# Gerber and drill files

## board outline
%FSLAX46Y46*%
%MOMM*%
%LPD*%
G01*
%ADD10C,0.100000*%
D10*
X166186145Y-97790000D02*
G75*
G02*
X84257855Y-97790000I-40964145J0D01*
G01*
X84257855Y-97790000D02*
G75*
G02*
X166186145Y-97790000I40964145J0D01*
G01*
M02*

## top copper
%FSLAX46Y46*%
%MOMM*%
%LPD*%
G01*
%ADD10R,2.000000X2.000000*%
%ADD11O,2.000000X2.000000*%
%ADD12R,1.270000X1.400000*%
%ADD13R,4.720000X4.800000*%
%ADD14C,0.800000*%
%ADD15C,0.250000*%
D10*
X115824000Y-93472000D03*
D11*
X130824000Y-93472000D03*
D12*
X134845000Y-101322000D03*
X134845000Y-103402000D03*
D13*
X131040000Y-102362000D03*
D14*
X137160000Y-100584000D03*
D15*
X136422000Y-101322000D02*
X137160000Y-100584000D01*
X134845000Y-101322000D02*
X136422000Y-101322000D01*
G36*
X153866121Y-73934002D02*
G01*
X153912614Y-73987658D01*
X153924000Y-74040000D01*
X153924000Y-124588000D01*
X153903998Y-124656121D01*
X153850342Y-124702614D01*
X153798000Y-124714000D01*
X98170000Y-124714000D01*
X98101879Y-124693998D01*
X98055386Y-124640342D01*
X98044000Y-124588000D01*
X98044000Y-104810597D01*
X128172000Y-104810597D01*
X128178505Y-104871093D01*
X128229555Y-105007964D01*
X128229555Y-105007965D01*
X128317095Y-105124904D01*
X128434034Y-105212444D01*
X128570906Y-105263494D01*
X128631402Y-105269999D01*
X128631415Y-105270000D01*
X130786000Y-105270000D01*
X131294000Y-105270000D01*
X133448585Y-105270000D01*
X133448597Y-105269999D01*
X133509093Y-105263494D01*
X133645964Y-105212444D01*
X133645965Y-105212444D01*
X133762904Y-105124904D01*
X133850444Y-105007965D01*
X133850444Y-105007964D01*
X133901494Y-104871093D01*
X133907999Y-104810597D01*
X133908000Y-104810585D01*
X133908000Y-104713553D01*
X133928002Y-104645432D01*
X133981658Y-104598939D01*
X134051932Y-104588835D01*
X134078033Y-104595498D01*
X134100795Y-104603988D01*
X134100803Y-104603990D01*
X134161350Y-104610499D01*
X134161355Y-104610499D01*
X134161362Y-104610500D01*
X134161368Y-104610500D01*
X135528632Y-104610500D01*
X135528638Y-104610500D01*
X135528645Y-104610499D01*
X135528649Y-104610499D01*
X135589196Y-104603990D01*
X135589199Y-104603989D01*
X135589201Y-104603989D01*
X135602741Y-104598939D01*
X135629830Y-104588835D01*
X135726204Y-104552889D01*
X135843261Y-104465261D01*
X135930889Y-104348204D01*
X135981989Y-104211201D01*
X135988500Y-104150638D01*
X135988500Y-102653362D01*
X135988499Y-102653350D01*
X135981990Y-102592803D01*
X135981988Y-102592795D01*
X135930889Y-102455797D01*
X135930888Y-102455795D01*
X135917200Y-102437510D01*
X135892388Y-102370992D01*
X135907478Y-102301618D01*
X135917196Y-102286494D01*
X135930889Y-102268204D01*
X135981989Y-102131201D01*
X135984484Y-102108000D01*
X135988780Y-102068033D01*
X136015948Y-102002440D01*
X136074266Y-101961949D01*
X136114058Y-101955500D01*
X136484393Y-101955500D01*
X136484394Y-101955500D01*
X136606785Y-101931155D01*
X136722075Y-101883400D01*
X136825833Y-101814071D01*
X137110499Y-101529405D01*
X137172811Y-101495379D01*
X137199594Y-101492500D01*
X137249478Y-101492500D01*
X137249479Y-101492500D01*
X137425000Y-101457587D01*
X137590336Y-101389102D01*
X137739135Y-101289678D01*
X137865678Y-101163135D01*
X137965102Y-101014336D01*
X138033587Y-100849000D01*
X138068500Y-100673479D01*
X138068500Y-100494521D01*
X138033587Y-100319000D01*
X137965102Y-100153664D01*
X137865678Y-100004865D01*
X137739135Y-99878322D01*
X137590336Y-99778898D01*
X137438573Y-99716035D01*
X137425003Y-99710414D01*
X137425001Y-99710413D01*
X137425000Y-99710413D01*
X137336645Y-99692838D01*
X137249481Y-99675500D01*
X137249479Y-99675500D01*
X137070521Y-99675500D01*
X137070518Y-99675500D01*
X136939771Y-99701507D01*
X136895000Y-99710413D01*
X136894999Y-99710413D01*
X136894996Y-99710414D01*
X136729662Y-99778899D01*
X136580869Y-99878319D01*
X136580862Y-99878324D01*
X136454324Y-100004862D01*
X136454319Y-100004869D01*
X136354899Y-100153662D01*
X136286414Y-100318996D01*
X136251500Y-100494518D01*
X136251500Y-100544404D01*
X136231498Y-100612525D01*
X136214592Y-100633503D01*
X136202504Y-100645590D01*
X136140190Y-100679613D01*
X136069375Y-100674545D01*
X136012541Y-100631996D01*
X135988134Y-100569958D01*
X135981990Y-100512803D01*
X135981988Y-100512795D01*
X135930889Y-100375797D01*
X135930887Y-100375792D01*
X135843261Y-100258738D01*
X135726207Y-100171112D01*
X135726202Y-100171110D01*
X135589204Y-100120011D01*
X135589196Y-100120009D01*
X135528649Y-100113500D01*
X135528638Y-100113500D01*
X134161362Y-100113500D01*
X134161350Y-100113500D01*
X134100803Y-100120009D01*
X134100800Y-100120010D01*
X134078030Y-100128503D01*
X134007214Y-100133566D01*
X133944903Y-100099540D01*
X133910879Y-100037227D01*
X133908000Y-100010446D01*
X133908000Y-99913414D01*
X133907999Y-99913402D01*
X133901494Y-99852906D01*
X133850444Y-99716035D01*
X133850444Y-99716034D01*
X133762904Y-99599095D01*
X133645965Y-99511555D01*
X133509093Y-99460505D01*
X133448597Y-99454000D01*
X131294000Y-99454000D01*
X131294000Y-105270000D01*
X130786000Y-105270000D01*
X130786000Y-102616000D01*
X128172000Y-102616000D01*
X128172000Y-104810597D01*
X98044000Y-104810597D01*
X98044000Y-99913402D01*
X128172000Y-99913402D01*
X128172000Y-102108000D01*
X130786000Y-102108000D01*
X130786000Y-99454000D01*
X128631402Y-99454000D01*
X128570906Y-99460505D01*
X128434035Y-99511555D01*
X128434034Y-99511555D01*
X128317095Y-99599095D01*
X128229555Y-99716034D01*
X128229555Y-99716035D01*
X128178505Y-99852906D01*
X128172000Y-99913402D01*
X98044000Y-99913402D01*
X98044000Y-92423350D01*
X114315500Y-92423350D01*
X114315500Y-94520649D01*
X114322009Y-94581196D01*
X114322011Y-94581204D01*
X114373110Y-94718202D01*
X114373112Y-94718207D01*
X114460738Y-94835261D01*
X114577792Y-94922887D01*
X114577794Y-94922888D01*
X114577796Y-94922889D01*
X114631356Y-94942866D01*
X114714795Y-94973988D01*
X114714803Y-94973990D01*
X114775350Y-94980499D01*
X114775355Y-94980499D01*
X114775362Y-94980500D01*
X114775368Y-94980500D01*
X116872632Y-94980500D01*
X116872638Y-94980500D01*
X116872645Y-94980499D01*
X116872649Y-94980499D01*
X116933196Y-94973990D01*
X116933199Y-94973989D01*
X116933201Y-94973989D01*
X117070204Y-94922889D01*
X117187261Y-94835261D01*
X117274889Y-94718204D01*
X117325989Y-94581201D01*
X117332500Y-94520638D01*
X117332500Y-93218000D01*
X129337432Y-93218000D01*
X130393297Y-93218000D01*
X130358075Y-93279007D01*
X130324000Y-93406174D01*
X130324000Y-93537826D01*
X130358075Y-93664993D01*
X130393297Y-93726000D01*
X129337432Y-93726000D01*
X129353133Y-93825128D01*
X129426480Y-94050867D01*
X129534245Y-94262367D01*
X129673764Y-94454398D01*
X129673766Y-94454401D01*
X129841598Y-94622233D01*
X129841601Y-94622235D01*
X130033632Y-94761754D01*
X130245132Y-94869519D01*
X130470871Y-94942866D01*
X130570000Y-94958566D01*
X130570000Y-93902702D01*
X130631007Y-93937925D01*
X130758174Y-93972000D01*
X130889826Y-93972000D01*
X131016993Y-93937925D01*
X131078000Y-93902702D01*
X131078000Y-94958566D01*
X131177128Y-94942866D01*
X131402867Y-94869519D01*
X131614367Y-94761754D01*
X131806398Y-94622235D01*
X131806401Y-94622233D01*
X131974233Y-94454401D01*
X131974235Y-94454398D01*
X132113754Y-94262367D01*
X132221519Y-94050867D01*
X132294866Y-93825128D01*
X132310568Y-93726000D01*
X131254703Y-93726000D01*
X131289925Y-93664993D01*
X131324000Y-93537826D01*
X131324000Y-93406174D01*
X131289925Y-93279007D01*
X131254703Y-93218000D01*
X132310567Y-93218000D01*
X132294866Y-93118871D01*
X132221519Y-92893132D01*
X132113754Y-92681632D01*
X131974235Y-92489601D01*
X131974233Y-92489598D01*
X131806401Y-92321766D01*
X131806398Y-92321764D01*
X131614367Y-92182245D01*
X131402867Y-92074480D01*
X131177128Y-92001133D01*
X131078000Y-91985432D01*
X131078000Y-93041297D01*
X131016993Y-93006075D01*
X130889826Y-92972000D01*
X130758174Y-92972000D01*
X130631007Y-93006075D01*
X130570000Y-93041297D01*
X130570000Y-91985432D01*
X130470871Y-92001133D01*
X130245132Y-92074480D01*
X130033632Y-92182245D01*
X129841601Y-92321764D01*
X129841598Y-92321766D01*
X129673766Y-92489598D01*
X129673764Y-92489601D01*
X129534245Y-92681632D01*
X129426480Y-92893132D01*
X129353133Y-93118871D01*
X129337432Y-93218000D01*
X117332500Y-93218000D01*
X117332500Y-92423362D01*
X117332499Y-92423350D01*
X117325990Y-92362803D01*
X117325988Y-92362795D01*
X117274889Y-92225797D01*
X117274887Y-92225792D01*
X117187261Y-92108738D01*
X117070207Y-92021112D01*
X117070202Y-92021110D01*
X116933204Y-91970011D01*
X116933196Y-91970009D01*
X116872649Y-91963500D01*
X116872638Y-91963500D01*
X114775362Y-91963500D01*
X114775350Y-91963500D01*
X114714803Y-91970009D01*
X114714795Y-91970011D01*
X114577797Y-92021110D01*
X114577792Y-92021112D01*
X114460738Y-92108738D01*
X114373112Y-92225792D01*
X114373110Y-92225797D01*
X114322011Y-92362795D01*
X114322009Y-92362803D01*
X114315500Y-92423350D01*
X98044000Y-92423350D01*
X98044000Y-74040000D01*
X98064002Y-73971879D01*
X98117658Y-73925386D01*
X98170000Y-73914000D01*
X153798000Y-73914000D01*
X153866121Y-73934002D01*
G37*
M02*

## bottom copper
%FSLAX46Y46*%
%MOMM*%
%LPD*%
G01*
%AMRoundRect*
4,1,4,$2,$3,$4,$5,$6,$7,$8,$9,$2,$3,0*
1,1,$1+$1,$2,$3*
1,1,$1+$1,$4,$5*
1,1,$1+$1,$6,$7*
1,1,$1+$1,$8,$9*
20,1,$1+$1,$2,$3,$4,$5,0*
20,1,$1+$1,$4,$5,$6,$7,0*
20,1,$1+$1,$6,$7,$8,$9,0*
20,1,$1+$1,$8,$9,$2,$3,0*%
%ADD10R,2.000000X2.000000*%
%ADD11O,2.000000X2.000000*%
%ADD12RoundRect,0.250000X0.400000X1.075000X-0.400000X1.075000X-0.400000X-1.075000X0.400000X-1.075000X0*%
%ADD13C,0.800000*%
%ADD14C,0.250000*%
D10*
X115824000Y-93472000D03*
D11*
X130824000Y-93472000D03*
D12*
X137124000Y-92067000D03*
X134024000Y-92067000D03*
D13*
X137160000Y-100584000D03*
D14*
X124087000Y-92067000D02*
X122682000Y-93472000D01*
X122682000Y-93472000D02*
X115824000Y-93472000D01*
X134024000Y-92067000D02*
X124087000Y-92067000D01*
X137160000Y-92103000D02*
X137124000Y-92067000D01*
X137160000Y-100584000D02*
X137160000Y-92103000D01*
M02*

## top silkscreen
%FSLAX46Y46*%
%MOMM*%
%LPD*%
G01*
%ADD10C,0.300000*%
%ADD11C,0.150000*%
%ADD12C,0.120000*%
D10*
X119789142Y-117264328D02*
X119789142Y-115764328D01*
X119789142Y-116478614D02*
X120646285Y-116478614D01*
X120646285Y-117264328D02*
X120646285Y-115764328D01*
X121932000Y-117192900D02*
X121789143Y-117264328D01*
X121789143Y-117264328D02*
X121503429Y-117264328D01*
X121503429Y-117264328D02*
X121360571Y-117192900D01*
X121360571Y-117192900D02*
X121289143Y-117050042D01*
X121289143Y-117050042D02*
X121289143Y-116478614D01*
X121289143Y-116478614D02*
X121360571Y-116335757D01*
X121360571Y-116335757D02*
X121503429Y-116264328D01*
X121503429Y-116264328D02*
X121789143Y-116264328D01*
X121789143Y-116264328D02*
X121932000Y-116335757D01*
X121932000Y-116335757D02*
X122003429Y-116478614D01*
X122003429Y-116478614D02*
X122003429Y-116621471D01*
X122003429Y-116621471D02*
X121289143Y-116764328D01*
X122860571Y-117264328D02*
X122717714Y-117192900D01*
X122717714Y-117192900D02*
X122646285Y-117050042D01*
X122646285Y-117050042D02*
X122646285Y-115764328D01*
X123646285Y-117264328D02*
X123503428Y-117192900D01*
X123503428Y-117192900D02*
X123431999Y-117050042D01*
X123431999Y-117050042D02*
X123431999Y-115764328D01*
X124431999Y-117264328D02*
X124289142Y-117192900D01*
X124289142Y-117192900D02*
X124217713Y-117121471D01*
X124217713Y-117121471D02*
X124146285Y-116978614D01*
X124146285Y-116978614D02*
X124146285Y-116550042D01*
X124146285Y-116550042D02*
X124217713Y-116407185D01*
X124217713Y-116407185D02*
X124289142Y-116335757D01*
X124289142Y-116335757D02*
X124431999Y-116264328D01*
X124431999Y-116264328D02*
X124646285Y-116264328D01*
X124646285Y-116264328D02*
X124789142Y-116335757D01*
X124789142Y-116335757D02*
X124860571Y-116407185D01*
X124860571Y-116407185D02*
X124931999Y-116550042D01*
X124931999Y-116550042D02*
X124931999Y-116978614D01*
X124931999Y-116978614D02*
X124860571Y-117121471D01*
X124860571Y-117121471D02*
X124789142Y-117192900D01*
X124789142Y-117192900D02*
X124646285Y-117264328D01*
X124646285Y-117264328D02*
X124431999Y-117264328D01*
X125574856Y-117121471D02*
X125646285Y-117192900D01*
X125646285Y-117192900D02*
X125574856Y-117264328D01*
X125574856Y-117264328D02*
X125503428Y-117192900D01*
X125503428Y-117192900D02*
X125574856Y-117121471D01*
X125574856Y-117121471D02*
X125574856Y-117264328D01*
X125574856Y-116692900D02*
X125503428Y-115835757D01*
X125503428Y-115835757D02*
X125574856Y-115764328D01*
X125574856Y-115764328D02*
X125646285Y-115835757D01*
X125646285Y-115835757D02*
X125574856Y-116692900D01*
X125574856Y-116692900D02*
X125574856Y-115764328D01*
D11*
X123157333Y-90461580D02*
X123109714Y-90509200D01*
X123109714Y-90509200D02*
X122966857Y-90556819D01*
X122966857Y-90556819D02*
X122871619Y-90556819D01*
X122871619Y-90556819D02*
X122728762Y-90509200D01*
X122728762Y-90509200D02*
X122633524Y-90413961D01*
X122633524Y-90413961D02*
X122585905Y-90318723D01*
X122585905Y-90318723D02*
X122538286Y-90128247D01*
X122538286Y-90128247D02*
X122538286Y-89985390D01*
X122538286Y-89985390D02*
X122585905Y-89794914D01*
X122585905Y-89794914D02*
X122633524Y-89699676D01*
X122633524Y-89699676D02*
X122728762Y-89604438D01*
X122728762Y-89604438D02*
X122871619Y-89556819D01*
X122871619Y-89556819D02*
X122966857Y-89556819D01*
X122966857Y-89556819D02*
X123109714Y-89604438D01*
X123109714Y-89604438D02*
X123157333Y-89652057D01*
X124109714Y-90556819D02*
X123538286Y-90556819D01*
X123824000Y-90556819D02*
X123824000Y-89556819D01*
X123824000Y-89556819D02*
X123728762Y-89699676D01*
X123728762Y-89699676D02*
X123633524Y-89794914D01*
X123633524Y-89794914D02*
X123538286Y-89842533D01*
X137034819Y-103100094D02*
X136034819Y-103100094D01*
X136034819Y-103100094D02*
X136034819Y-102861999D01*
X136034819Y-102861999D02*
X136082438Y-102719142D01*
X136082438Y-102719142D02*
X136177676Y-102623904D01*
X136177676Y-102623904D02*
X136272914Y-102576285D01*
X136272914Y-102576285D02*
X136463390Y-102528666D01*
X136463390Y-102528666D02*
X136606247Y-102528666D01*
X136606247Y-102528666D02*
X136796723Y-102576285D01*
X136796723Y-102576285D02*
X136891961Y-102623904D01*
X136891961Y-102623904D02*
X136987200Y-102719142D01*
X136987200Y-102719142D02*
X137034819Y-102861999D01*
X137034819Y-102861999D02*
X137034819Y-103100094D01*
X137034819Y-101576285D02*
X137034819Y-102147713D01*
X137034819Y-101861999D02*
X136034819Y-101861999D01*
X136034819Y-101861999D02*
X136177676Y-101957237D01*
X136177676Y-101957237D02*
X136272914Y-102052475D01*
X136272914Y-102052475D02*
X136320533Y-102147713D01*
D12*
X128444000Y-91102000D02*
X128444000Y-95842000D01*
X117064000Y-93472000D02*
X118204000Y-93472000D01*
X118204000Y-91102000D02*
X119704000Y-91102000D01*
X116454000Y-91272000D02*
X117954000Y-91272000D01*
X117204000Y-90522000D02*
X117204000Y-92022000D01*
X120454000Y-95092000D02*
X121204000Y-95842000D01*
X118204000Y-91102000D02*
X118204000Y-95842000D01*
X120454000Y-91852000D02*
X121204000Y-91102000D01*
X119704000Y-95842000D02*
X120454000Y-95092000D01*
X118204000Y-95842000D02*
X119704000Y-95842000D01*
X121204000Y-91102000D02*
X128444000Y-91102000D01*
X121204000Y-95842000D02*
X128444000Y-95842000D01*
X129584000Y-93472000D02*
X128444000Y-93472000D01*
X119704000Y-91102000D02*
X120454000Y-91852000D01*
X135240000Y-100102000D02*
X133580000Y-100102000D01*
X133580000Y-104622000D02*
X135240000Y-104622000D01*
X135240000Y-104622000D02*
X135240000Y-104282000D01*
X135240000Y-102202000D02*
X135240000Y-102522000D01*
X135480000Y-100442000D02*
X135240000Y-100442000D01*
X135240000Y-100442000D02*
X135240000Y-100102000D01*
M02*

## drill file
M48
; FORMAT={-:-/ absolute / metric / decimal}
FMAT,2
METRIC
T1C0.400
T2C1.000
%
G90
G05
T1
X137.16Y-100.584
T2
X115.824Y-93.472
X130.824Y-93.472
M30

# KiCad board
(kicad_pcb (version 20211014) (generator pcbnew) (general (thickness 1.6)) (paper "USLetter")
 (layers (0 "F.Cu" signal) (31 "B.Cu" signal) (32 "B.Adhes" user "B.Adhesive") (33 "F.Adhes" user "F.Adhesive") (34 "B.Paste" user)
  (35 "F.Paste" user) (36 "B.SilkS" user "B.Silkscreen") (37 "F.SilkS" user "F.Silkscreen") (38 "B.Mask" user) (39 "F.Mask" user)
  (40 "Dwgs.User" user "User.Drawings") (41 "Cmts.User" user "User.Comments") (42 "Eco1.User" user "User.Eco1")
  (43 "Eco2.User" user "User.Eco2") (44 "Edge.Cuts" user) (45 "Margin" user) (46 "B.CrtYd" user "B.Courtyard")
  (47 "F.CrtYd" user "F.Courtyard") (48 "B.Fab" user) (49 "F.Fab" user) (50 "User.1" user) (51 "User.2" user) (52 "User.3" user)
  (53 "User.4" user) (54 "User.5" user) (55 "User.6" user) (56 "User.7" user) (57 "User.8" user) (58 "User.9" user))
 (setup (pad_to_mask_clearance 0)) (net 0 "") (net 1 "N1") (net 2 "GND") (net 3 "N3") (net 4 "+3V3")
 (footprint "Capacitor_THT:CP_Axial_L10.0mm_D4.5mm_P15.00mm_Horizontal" (layer "F.Cu") (at 115.824 93.472)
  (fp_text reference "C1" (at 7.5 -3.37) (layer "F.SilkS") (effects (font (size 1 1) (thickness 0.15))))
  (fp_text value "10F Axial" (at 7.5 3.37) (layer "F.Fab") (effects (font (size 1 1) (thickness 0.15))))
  (fp_line (start 12.62 -2.37) (end 12.62 2.37) (layer "F.SilkS") (width 0.12))
  (fp_line (start 1.24 0) (end 2.38 0) (layer "F.SilkS") (width 0.12))
  (fp_line (start 2.38 -2.37) (end 3.88 -2.37) (layer "F.SilkS") (width 0.12))
  (fp_line (start 0.63 -2.2) (end 2.13 -2.2) (layer "F.SilkS") (width 0.12))
  (fp_line (start 1.38 -2.95) (end 1.38 -1.45) (layer "F.SilkS") (width 0.12))
  (fp_line (start 4.63 1.62) (end 5.38 2.37) (layer "F.SilkS") (width 0.12))
  (fp_line (start 2.38 -2.37) (end 2.38 2.37) (layer "F.SilkS") (width 0.12))
  (fp_line (start 4.63 -1.62) (end 5.38 -2.37) (layer "F.SilkS") (width 0.12))
  (fp_line (start 3.88 2.37) (end 4.63 1.62) (layer "F.SilkS") (width 0.12))
  (fp_line (start 2.38 2.37) (end 3.88 2.37) (layer "F.SilkS") (width 0.12))
  (fp_line (start 5.38 -2.37) (end 12.62 -2.37) (layer "F.SilkS") (width 0.12))
  (fp_line (start 5.38 2.37) (end 12.62 2.37) (layer "F.SilkS") (width 0.12))
  (fp_line (start 13.76 0) (end 12.62 0) (layer "F.SilkS") (width 0.12))
  (fp_line (start 3.88 -2.37) (end 4.63 -1.62) (layer "F.SilkS") (width 0.12))
  (pad "1" thru_hole rect (at 0 0) (size 2 2) (drill 1) (layers *.Cu *.Mask) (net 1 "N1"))
  (pad "2" thru_hole oval (at 15 0) (size 2 2) (drill 1) (layers *.Cu *.Mask) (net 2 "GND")))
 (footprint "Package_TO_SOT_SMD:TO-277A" (layer "F.Cu") (at 132.08 102.362 -90)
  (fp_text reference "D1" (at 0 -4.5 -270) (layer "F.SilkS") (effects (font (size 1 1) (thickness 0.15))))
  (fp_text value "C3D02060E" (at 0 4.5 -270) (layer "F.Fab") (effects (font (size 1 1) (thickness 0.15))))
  (fp_line (start -2.26 -3.16) (end -2.26 -1.5) (layer "F.SilkS") (width 0.12))
  (fp_line (start 2.26 -1.5) (end 2.26 -3.16) (layer "F.SilkS") (width 0.12))
  (fp_line (start 2.26 -3.16) (end 1.92 -3.16) (layer "F.SilkS") (width 0.12))
  (fp_line (start -0.16 -3.16) (end 0.16 -3.16) (layer "F.SilkS") (width 0.12))
  (fp_line (start -1.92 -3.4) (end -1.92 -3.16) (layer "F.SilkS") (width 0.12))
  (fp_line (start -1.92 -3.16) (end -2.26 -3.16) (layer "F.SilkS") (width 0.12))
  (pad "" smd rect (at -1.7 1.04 270) (size 1.25 1.2) (layers "F.Paste"))
  (pad "" smd rect (at 1.7 -0.65 270) (size 1.25 1.2) (layers "F.Paste"))
  (pad "" smd rect (at 1.7 1.04 270) (size 1.25 1.2) (layers "F.Paste"))
  (pad "" smd rect (at 0 2.7 270) (size 1.25 1.2) (layers "F.Paste"))
  (pad "" smd rect (at 0 1.04 270) (size 1.25 1.2) (layers "F.Paste"))
  (pad "" smd rect (at 0 -0.65 270) (size 1.25 1.2) (layers "F.Paste"))
  (pad "" smd rect (at 1.7 2.7 270) (size 1.25 1.2) (layers "F.Paste"))
  (pad "" smd rect (at -1.7 -0.65 90) (size 1.25 1.2) (layers "F.Paste"))
  (pad "" smd rect (at -1.7 2.7 270) (size 1.25 1.2) (layers "F.Paste"))
  (pad "1" smd rect (at -1.04 -2.765 270) (size 1.4 1.27) (layers "F.Cu" "F.Paste" "F.Mask") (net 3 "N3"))
  (pad "2" smd rect (at 1.04 -2.765 270) (size 1.4 1.27) (layers "F.Cu" "F.Paste" "F.Mask") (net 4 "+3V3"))
  (pad "3" smd rect (at 0 1.04 270) (size 4.8 4.72) (layers "F.Cu" "F.Mask") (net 2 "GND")))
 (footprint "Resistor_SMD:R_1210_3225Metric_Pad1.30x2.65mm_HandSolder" (layer "B.Cu") (at 135.574 92.067 180)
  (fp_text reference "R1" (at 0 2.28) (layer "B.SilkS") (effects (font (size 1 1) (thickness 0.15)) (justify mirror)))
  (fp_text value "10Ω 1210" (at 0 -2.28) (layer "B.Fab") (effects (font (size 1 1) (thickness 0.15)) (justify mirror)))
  (pad "1" smd roundrect (at -1.55 0 180) (size 1.3 2.65) (layers "B.Cu" "B.Paste" "B.Mask") (roundrect_rratio 0.192308) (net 3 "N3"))
  (pad "2" smd roundrect (at 1.55 0 180) (size 1.3 2.65) (layers "B.Cu" "B.Paste" "B.Mask") (roundrect_rratio 0.192308) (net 1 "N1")))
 (gr_circle (center 125.222 97.79) (end 164.084 84.836) (layer "Edge.Cuts") (width 0.1) (fill none))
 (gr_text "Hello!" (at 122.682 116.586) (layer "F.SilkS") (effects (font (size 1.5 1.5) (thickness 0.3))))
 (segment (start 124.087 92.067) (end 122.682 93.472) (width 0.25) (layer "B.Cu") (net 1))
 (segment (start 122.682 93.472) (end 115.824 93.472) (width 0.25) (layer "B.Cu") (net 1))
 (segment (start 134.024 92.067) (end 124.087 92.067) (width 0.25) (layer "B.Cu") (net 1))
 (segment (start 136.422 101.322) (end 137.16 100.584) (width 0.25) (layer "F.Cu") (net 3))
 (segment (start 134.845 101.322) (end 136.422 101.322) (width 0.25) (layer "F.Cu") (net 3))
 (via (at 137.16 100.584) (size 0.8) (drill 0.4) (layers "F.Cu" "B.Cu") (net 3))
 (segment (start 137.16 92.103) (end 137.124 92.067) (width 0.25) (layer "B.Cu") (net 3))
 (segment (start 137.16 100.584) (end 137.16 92.103) (width 0.25) (layer "B.Cu") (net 3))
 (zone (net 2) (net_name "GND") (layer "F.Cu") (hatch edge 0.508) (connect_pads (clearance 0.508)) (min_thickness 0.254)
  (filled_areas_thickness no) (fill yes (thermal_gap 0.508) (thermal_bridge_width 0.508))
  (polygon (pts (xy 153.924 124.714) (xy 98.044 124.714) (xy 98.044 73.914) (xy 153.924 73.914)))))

